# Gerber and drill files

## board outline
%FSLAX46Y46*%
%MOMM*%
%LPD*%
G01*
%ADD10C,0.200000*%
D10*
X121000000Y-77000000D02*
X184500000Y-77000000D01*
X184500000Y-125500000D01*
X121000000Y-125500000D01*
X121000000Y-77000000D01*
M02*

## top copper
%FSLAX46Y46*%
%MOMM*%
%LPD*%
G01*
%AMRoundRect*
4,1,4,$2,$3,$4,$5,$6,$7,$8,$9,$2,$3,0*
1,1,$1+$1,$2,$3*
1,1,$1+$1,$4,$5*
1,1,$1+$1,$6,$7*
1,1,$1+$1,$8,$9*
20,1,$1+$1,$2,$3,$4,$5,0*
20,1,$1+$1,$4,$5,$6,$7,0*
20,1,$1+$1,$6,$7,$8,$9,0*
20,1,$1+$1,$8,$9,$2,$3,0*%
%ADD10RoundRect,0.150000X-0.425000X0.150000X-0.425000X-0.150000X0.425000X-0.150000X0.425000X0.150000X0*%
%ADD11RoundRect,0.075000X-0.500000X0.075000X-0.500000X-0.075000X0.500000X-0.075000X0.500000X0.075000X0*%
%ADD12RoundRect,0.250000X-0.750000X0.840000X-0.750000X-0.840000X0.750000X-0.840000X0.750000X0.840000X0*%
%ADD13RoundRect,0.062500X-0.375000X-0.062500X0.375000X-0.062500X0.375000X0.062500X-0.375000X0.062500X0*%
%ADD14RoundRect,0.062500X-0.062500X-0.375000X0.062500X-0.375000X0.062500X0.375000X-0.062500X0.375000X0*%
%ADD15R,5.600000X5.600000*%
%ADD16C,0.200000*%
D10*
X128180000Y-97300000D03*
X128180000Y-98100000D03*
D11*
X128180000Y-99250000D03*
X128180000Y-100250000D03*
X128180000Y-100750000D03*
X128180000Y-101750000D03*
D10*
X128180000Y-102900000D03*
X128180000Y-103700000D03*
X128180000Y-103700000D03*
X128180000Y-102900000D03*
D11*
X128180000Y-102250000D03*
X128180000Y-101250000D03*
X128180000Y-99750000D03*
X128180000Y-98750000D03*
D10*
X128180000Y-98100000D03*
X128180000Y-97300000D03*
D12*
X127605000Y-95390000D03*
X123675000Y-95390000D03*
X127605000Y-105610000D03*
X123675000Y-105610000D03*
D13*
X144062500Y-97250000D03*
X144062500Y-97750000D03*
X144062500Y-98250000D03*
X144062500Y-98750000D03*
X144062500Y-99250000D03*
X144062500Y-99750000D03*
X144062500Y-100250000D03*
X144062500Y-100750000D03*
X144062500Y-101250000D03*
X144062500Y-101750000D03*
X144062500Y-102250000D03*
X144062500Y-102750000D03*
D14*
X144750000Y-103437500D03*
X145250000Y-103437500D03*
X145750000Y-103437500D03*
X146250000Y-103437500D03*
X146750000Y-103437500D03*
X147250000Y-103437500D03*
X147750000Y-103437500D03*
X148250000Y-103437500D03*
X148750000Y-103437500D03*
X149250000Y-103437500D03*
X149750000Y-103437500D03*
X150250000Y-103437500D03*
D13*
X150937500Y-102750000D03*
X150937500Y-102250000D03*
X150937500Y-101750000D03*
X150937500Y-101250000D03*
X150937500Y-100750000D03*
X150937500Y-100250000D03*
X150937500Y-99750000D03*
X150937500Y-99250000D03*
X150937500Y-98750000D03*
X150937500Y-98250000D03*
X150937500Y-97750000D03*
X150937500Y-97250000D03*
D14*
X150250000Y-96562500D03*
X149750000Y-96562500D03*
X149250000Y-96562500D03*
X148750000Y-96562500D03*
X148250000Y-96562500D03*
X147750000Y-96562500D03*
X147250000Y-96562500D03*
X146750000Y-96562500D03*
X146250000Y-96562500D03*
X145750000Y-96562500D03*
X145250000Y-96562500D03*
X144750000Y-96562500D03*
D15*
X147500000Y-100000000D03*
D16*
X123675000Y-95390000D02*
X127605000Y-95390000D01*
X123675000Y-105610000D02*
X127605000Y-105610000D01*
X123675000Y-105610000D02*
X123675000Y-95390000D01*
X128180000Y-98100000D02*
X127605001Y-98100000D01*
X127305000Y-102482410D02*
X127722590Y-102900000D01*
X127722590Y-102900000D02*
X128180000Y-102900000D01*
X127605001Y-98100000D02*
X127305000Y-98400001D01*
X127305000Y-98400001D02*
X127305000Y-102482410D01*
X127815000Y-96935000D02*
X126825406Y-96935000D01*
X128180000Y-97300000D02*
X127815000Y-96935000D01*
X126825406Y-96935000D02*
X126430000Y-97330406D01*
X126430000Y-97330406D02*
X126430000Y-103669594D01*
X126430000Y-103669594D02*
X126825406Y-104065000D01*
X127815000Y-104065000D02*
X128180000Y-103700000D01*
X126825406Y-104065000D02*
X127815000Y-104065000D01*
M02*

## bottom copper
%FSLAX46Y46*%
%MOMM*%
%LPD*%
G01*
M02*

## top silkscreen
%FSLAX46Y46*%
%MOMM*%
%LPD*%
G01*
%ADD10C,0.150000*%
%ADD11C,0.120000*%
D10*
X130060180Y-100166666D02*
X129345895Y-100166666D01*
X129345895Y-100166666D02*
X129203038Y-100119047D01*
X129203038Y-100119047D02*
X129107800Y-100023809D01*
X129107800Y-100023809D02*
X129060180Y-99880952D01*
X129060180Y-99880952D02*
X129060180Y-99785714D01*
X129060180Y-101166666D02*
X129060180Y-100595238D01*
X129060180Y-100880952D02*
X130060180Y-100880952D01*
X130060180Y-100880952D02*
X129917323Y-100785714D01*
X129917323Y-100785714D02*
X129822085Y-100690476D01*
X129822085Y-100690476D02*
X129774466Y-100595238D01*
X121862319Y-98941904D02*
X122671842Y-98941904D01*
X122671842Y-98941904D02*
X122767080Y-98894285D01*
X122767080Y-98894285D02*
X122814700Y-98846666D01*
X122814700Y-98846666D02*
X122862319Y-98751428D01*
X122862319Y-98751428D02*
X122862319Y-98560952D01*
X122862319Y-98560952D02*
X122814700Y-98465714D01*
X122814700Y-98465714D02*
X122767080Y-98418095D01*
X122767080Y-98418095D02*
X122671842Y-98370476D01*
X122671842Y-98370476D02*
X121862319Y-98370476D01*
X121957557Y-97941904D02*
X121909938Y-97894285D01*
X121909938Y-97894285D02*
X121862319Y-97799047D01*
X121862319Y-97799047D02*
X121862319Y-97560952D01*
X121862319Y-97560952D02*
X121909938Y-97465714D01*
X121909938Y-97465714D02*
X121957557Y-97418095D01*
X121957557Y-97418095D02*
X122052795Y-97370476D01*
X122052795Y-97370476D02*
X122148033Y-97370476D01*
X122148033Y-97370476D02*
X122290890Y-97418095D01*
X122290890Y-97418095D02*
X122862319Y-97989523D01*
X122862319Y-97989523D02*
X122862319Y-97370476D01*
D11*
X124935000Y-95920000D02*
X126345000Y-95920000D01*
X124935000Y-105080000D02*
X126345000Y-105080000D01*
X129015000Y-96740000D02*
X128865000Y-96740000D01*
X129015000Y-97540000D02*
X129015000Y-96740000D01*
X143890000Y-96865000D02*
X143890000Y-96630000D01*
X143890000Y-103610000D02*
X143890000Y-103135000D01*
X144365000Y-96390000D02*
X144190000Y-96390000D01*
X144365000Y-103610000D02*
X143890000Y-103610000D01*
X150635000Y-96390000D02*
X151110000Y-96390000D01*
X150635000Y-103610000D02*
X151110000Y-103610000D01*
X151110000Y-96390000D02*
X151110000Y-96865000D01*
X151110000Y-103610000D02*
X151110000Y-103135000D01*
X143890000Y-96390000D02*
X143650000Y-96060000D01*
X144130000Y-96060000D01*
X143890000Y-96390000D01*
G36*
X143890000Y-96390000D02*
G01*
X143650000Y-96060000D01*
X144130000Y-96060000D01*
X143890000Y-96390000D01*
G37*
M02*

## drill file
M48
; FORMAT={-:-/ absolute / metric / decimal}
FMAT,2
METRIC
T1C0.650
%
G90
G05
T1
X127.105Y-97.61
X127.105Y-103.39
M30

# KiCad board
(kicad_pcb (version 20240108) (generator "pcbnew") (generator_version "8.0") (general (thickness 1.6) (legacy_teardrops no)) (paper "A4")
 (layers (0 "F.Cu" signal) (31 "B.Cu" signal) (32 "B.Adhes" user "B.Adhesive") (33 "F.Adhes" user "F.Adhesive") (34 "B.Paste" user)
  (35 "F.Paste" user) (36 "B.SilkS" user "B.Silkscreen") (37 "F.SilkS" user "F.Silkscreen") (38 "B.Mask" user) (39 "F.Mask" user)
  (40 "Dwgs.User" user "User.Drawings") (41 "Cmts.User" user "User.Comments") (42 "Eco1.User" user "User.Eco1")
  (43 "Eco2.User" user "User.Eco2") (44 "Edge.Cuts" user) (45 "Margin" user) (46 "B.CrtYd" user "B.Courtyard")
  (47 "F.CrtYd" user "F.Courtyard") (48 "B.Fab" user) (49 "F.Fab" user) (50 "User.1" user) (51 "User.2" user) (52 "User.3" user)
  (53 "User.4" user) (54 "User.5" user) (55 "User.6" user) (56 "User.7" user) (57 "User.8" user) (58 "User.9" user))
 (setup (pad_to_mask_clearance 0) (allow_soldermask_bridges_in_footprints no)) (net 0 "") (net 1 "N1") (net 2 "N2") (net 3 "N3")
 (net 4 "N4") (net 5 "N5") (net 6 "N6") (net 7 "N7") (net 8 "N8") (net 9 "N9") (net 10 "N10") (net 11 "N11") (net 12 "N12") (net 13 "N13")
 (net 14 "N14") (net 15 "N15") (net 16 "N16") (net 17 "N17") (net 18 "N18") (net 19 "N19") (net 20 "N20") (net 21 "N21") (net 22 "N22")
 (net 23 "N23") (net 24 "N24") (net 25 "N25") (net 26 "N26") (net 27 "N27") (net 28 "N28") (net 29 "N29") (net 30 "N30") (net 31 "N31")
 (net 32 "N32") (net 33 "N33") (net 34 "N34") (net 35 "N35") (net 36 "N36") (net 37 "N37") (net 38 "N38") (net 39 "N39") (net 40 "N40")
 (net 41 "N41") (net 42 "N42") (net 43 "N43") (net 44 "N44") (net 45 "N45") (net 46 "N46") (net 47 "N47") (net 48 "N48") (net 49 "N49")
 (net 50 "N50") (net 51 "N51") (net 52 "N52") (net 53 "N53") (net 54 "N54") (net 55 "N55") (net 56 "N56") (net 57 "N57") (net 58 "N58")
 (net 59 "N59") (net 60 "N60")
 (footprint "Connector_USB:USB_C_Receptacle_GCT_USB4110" (layer "F.Cu") (at 124.5 100.5 -90)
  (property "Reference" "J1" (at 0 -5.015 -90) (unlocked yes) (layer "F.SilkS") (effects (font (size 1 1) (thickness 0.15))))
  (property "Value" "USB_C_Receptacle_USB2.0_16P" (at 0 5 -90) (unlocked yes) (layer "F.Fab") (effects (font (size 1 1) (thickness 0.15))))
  (fp_line (start -4.58 -0.435) (end -4.58 -1.845) (stroke (width 0.12) (type default)) (layer "F.SilkS"))
  (fp_line (start 4.58 -0.435) (end 4.58 -1.845) (stroke (width 0.12) (type default)) (layer "F.SilkS"))
  (fp_line (start -3.76 -4.515) (end -3.76 -4.365) (stroke (width 0.12) (type default)) (layer "F.SilkS"))
  (fp_line (start -2.96 -4.515) (end -3.76 -4.515) (stroke (width 0.12) (type default)) (layer "F.SilkS"))
  (pad "" np_thru_hole circle (at -2.89 -2.605 270) (size 0.65 0.65) (drill 0.65) (layers "F&B.Cu" "*.Mask"))
  (pad "" np_thru_hole circle (at 2.89 -2.605 270) (size 0.65 0.65) (drill 0.65) (layers "F&B.Cu" "*.Mask"))
  (pad "A1" smd roundrect (at -3.2 -3.68 270) (size 0.6 1.15) (layers "F.Cu" "F.Paste" "F.Mask") (roundrect_rratio 0.25) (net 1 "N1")
   (thermal_bridge_angle 45))
  (pad "A4" smd roundrect (at -2.4 -3.68 270) (size 0.6 1.15) (layers "F.Cu" "F.Paste" "F.Mask") (roundrect_rratio 0.25) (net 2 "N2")
   (thermal_bridge_angle 45))
  (pad "A5" smd roundrect (at -1.25 -3.68 270) (size 0.3 1.15) (layers "F.Cu" "F.Paste" "F.Mask") (roundrect_rratio 0.25) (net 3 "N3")
   (thermal_bridge_angle 45))
  (pad "A6" smd roundrect (at -0.25 -3.68 270) (size 0.3 1.15) (layers "F.Cu" "F.Paste" "F.Mask") (roundrect_rratio 0.25) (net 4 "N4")
   (thermal_bridge_angle 45))
  (pad "A7" smd roundrect (at 0.25 -3.68 270) (size 0.3 1.15) (layers "F.Cu" "F.Paste" "F.Mask") (roundrect_rratio 0.25) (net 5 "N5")
   (thermal_bridge_angle 45))
  (pad "A8" smd roundrect (at 1.25 -3.68 270) (size 0.3 1.15) (layers "F.Cu" "F.Paste" "F.Mask") (roundrect_rratio 0.25) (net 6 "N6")
   (thermal_bridge_angle 45))
  (pad "A9" smd roundrect (at 2.4 -3.68 270) (size 0.6 1.15) (layers "F.Cu" "F.Paste" "F.Mask") (roundrect_rratio 0.25) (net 2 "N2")
   (thermal_bridge_angle 45))
  (pad "A12" smd roundrect (at 3.2 -3.68 270) (size 0.6 1.15) (layers "F.Cu" "F.Paste" "F.Mask") (roundrect_rratio 0.25) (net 1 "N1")
   (thermal_bridge_angle 45))
  (pad "B1" smd roundrect (at 3.2 -3.68 270) (size 0.6 1.15) (layers "F.Cu" "F.Paste" "F.Mask") (roundrect_rratio 0.25) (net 1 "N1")
   (thermal_bridge_angle 45))
  (pad "B4" smd roundrect (at 2.4 -3.68 270) (size 0.6 1.15) (layers "F.Cu" "F.Paste" "F.Mask") (roundrect_rratio 0.25) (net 2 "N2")
   (thermal_bridge_angle 45))
  (pad "B5" smd roundrect (at 1.75 -3.68 270) (size 0.3 1.15) (layers "F.Cu" "F.Paste" "F.Mask") (roundrect_rratio 0.25) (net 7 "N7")
   (thermal_bridge_angle 45))
  (pad "B6" smd roundrect (at 0.75 -3.68 270) (size 0.3 1.15) (layers "F.Cu" "F.Paste" "F.Mask") (roundrect_rratio 0.25) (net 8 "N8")
   (thermal_bridge_angle 45))
  (pad "B7" smd roundrect (at -0.75 -3.68 270) (size 0.3 1.15) (layers "F.Cu" "F.Paste" "F.Mask") (roundrect_rratio 0.25) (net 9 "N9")
   (thermal_bridge_angle 45))
  (pad "B8" smd roundrect (at -1.75 -3.68 270) (size 0.3 1.15) (layers "F.Cu" "F.Paste" "F.Mask") (roundrect_rratio 0.25) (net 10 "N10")
   (thermal_bridge_angle 45))
  (pad "B9" smd roundrect (at -2.4 -3.68 270) (size 0.6 1.15) (layers "F.Cu" "F.Paste" "F.Mask") (roundrect_rratio 0.25) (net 2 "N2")
   (thermal_bridge_angle 45))
  (pad "B12" smd roundrect (at -3.2 -3.68 270) (size 0.6 1.15) (layers "F.Cu" "F.Paste" "F.Mask") (roundrect_rratio 0.25) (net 1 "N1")
   (thermal_bridge_angle 45))
  (pad "S1" smd roundrect (at -5.11 -3.105 270) (size 2.18 2) (layers "F.Cu" "F.Paste" "F.Mask") (roundrect_rratio 0.125) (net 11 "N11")
   (thermal_bridge_angle 45))
  (pad "S1" smd roundrect (at -5.11 0.825 270) (size 2.18 2) (layers "F.Cu" "F.Paste" "F.Mask") (roundrect_rratio 0.125) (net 11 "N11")
   (thermal_bridge_angle 45))
  (pad "S1" smd roundrect (at 5.11 -3.105 270) (size 2.18 2) (layers "F.Cu" "F.Paste" "F.Mask") (roundrect_rratio 0.125) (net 11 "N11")
   (thermal_bridge_angle 45))
  (pad "S1" smd roundrect (at 5.11 0.825 270) (size 2.18 2) (layers "F.Cu" "F.Paste" "F.Mask") (roundrect_rratio 0.125) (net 11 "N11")
   (thermal_bridge_angle 45)))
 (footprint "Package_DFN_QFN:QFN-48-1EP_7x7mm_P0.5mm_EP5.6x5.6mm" (layer "F.Cu") (at 147.5 100)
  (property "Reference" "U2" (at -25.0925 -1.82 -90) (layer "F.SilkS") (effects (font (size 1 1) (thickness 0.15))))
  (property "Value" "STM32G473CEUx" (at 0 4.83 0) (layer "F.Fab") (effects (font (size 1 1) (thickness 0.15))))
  (fp_line (start -3.61 -3.135) (end -3.61 -3.37) (stroke (width 0.12) (type solid)) (layer "F.SilkS"))
  (fp_line (start -3.61 3.61) (end -3.61 3.135) (stroke (width 0.12) (type solid)) (layer "F.SilkS"))
  (fp_line (start -3.135 -3.61) (end -3.31 -3.61) (stroke (width 0.12) (type solid)) (layer "F.SilkS"))
  (fp_line (start -3.135 3.61) (end -3.61 3.61) (stroke (width 0.12) (type solid)) (layer "F.SilkS"))
  (fp_line (start 3.135 -3.61) (end 3.61 -3.61) (stroke (width 0.12) (type solid)) (layer "F.SilkS"))
  (fp_line (start 3.135 3.61) (end 3.61 3.61) (stroke (width 0.12) (type solid)) (layer "F.SilkS"))
  (fp_line (start 3.61 -3.61) (end 3.61 -3.135) (stroke (width 0.12) (type solid)) (layer "F.SilkS"))
  (fp_line (start 3.61 3.61) (end 3.61 3.135) (stroke (width 0.12) (type solid)) (layer "F.SilkS"))
  (fp_poly
   (pts (xy -3.61 -3.61) (xy -3.85 -3.94) (xy -3.37 -3.94) (xy -3.61 -3.61)) (stroke (width 0.12) (type solid)) (fill solid)
   (layer "F.SilkS"))
  (pad "" smd roundrect (at -2.1 -2.1) (size 1.13 1.13) (layers "F.Paste") (roundrect_rratio 0.221239))
  (pad "" smd roundrect (at -2.1 -0.7) (size 1.13 1.13) (layers "F.Paste") (roundrect_rratio 0.221239))
  (pad "" smd roundrect (at -2.1 0.7) (size 1.13 1.13) (layers "F.Paste") (roundrect_rratio 0.221239))
  (pad "" smd roundrect (at -2.1 2.1) (size 1.13 1.13) (layers "F.Paste") (roundrect_rratio 0.221239))
  (pad "" smd roundrect (at -0.7 -2.1) (size 1.13 1.13) (layers "F.Paste") (roundrect_rratio 0.221239))
  (pad "" smd roundrect (at -0.7 -0.7) (size 1.13 1.13) (layers "F.Paste") (roundrect_rratio 0.221239))
  (pad "" smd roundrect (at -0.7 0.7) (size 1.13 1.13) (layers "F.Paste") (roundrect_rratio 0.221239))
  (pad "" smd roundrect (at -0.7 2.1) (size 1.13 1.13) (layers "F.Paste") (roundrect_rratio 0.221239))
  (pad "" smd roundrect (at 0.7 -2.1) (size 1.13 1.13) (layers "F.Paste") (roundrect_rratio 0.221239))
  (pad "" smd roundrect (at 0.7 -0.7) (size 1.13 1.13) (layers "F.Paste") (roundrect_rratio 0.221239))
  (pad "" smd roundrect (at 0.7 0.7) (size 1.13 1.13) (layers "F.Paste") (roundrect_rratio 0.221239))
  (pad "" smd roundrect (at 0.7 2.1) (size 1.13 1.13) (layers "F.Paste") (roundrect_rratio 0.221239))
  (pad "" smd roundrect (at 2.1 -2.1) (size 1.13 1.13) (layers "F.Paste") (roundrect_rratio 0.221239))
  (pad "" smd roundrect (at 2.1 -0.7) (size 1.13 1.13) (layers "F.Paste") (roundrect_rratio 0.221239))
  (pad "" smd roundrect (at 2.1 0.7) (size 1.13 1.13) (layers "F.Paste") (roundrect_rratio 0.221239))
  (pad "" smd roundrect (at 2.1 2.1) (size 1.13 1.13) (layers "F.Paste") (roundrect_rratio 0.221239))
  (pad "1" smd roundrect (at -3.4375 -2.75) (size 0.875 0.25) (layers "F.Cu" "F.Paste" "F.Mask") (roundrect_rratio 0.25) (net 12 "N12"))
  (pad "2" smd roundrect (at -3.4375 -2.25) (size 0.875 0.25) (layers "F.Cu" "F.Paste" "F.Mask") (roundrect_rratio 0.25) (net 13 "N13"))
  (pad "3" smd roundrect (at -3.4375 -1.75) (size 0.875 0.25) (layers "F.Cu" "F.Paste" "F.Mask") (roundrect_rratio 0.25) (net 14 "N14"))
  (pad "4" smd roundrect (at -3.4375 -1.25) (size 0.875 0.25) (layers "F.Cu" "F.Paste" "F.Mask") (roundrect_rratio 0.25) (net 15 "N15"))
  (pad "5" smd roundrect (at -3.4375 -0.75) (size 0.875 0.25) (layers "F.Cu" "F.Paste" "F.Mask") (roundrect_rratio 0.25) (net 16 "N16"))
  (pad "6" smd roundrect (at -3.4375 -0.25) (size 0.875 0.25) (layers "F.Cu" "F.Paste" "F.Mask") (roundrect_rratio 0.25) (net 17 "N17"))
  (pad "7" smd roundrect (at -3.4375 0.25) (size 0.875 0.25) (layers "F.Cu" "F.Paste" "F.Mask") (roundrect_rratio 0.25) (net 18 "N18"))
  (pad "8" smd roundrect (at -3.4375 0.75) (size 0.875 0.25) (layers "F.Cu" "F.Paste" "F.Mask") (roundrect_rratio 0.25) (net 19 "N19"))
  (pad "9" smd roundrect (at -3.4375 1.25) (size 0.875 0.25) (layers "F.Cu" "F.Paste" "F.Mask") (roundrect_rratio 0.25) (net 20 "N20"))
  (pad "10" smd roundrect (at -3.4375 1.75) (size 0.875 0.25) (layers "F.Cu" "F.Paste" "F.Mask") (roundrect_rratio 0.25) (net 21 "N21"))
  (pad "11" smd roundrect (at -3.4375 2.25) (size 0.875 0.25) (layers "F.Cu" "F.Paste" "F.Mask") (roundrect_rratio 0.25) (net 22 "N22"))
  (pad "12" smd roundrect (at -3.4375 2.75) (size 0.875 0.25) (layers "F.Cu" "F.Paste" "F.Mask") (roundrect_rratio 0.25) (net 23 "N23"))
  (pad "13" smd roundrect (at -2.75 3.4375) (size 0.25 0.875) (layers "F.Cu" "F.Paste" "F.Mask") (roundrect_rratio 0.25) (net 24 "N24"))
  (pad "14" smd roundrect (at -2.25 3.4375) (size 0.25 0.875) (layers "F.Cu" "F.Paste" "F.Mask") (roundrect_rratio 0.25) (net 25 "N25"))
  (pad "15" smd roundrect (at -1.75 3.4375) (size 0.25 0.875) (layers "F.Cu" "F.Paste" "F.Mask") (roundrect_rratio 0.25) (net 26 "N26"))
  (pad "16" smd roundrect (at -1.25 3.4375) (size 0.25 0.875) (layers "F.Cu" "F.Paste" "F.Mask") (roundrect_rratio 0.25) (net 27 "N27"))
  (pad "17" smd roundrect (at -0.75 3.4375) (size 0.25 0.875) (layers "F.Cu" "F.Paste" "F.Mask") (roundrect_rratio 0.25) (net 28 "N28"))
  (pad "18" smd roundrect (at -0.25 3.4375) (size 0.25 0.875) (layers "F.Cu" "F.Paste" "F.Mask") (roundrect_rratio 0.25) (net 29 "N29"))
  (pad "19" smd roundrect (at 0.25 3.4375) (size 0.25 0.875) (layers "F.Cu" "F.Paste" "F.Mask") (roundrect_rratio 0.25) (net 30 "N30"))
  (pad "20" smd roundrect (at 0.75 3.4375) (size 0.25 0.875) (layers "F.Cu" "F.Paste" "F.Mask") (roundrect_rratio 0.25) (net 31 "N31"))
  (pad "21" smd roundrect (at 1.25 3.4375) (size 0.25 0.875) (layers "F.Cu" "F.Paste" "F.Mask") (roundrect_rratio 0.25) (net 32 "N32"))
  (pad "22" smd roundrect (at 1.75 3.4375) (size 0.25 0.875) (layers "F.Cu" "F.Paste" "F.Mask") (roundrect_rratio 0.25) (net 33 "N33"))
  (pad "23" smd roundrect (at 2.25 3.4375) (size 0.25 0.875) (layers "F.Cu" "F.Paste" "F.Mask") (roundrect_rratio 0.25) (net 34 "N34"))
  (pad "24" smd roundrect (at 2.75 3.4375) (size 0.25 0.875) (layers "F.Cu" "F.Paste" "F.Mask") (roundrect_rratio 0.25) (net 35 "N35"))
  (pad "25" smd roundrect (at 3.4375 2.75) (size 0.875 0.25) (layers "F.Cu" "F.Paste" "F.Mask") (roundrect_rratio 0.25) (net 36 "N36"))
  (pad "26" smd roundrect (at 3.4375 2.25) (size 0.875 0.25) (layers "F.Cu" "F.Paste" "F.Mask") (roundrect_rratio 0.25) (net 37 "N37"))
  (pad "27" smd roundrect (at 3.4375 1.75) (size 0.875 0.25) (layers "F.Cu" "F.Paste" "F.Mask") (roundrect_rratio 0.25) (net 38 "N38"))
  (pad "28" smd roundrect (at 3.4375 1.25) (size 0.875 0.25) (layers "F.Cu" "F.Paste" "F.Mask") (roundrect_rratio 0.25) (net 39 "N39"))
  (pad "29" smd roundrect (at 3.4375 0.75) (size 0.875 0.25) (layers "F.Cu" "F.Paste" "F.Mask") (roundrect_rratio 0.25) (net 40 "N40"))
  (pad "30" smd roundrect (at 3.4375 0.25) (size 0.875 0.25) (layers "F.Cu" "F.Paste" "F.Mask") (roundrect_rratio 0.25) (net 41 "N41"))
  (pad "31" smd roundrect (at 3.4375 -0.25) (size 0.875 0.25) (layers "F.Cu" "F.Paste" "F.Mask") (roundrect_rratio 0.25) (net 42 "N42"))
  (pad "32" smd roundrect (at 3.4375 -0.75) (size 0.875 0.25) (layers "F.Cu" "F.Paste" "F.Mask") (roundrect_rratio 0.25) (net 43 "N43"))
  (pad "33" smd roundrect (at 3.4375 -1.25) (size 0.875 0.25) (layers "F.Cu" "F.Paste" "F.Mask") (roundrect_rratio 0.25) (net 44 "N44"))
  (pad "34" smd roundrect (at 3.4375 -1.75) (size 0.875 0.25) (layers "F.Cu" "F.Paste" "F.Mask") (roundrect_rratio 0.25) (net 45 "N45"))
  (pad "35" smd roundrect (at 3.4375 -2.25) (size 0.875 0.25) (layers "F.Cu" "F.Paste" "F.Mask") (roundrect_rratio 0.25) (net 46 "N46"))
  (pad "36" smd roundrect (at 3.4375 -2.75) (size 0.875 0.25) (layers "F.Cu" "F.Paste" "F.Mask") (roundrect_rratio 0.25) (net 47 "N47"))
  (pad "37" smd roundrect (at 2.75 -3.4375) (size 0.25 0.875) (layers "F.Cu" "F.Paste" "F.Mask") (roundrect_rratio 0.25) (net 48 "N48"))
  (pad "38" smd roundrect (at 2.25 -3.4375) (size 0.25 0.875) (layers "F.Cu" "F.Paste" "F.Mask") (roundrect_rratio 0.25) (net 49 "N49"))
  (pad "39" smd roundrect (at 1.75 -3.4375) (size 0.25 0.875) (layers "F.Cu" "F.Paste" "F.Mask") (roundrect_rratio 0.25) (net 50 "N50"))
  (pad "40" smd roundrect (at 1.25 -3.4375) (size 0.25 0.875) (layers "F.Cu" "F.Paste" "F.Mask") (roundrect_rratio 0.25) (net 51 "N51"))
  (pad "41" smd roundrect (at 0.75 -3.4375) (size 0.25 0.875) (layers "F.Cu" "F.Paste" "F.Mask") (roundrect_rratio 0.25) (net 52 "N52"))
  (pad "42" smd roundrect (at 0.25 -3.4375) (size 0.25 0.875) (layers "F.Cu" "F.Paste" "F.Mask") (roundrect_rratio 0.25) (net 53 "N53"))
  (pad "43" smd roundrect (at -0.25 -3.4375) (size 0.25 0.875) (layers "F.Cu" "F.Paste" "F.Mask") (roundrect_rratio 0.25) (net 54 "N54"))
  (pad "44" smd roundrect (at -0.75 -3.4375) (size 0.25 0.875) (layers "F.Cu" "F.Paste" "F.Mask") (roundrect_rratio 0.25) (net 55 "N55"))
  (pad "45" smd roundrect (at -1.25 -3.4375) (size 0.25 0.875) (layers "F.Cu" "F.Paste" "F.Mask") (roundrect_rratio 0.25) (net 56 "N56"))
  (pad "46" smd roundrect (at -1.75 -3.4375) (size 0.25 0.875) (layers "F.Cu" "F.Paste" "F.Mask") (roundrect_rratio 0.25) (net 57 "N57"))
  (pad "47" smd roundrect (at -2.25 -3.4375) (size 0.25 0.875) (layers "F.Cu" "F.Paste" "F.Mask") (roundrect_rratio 0.25) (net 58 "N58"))
  (pad "48" smd roundrect (at -2.75 -3.4375) (size 0.25 0.875) (layers "F.Cu" "F.Paste" "F.Mask") (roundrect_rratio 0.25) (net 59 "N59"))
  (pad "49" smd rect (at 0 0) (size 5.6 5.6) (layers "F.Cu" "F.Mask") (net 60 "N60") (zone_connect 2)))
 (gr_rect (start 121 77) (end 184.5 125.5) (stroke (width 0.2) (type default)) (fill none) (layer "Edge.Cuts"))
 (segment (start 123.675 95.39) (end 127.605 95.39) (width 0.2) (layer "F.Cu") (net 11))
 (segment (start 123.675 105.61) (end 127.605 105.61) (width 0.2) (layer "F.Cu") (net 11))
 (segment (start 123.675 105.61) (end 123.675 95.39) (width 0.2) (layer "F.Cu") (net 11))
 (segment (start 128.18 98.1) (end 127.605001 98.1) (width 0.2) (layer "F.Cu") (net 2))
 (segment (start 127.305 102.48241) (end 127.72259 102.9) (width 0.2) (layer "F.Cu") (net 2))
 (segment (start 127.72259 102.9) (end 128.18 102.9) (width 0.2) (layer "F.Cu") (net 2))
 (segment (start 127.605001 98.1) (end 127.305 98.400001) (width 0.2) (layer "F.Cu") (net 2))
 (segment (start 127.305 98.400001) (end 127.305 102.48241) (width 0.2) (layer "F.Cu") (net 2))
 (segment (start 127.815 96.935) (end 126.825406 96.935) (width 0.2) (layer "F.Cu") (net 1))
 (segment (start 128.18 97.3) (end 127.815 96.935) (width 0.2) (layer "F.Cu") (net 1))
 (segment (start 126.825406 96.935) (end 126.43 97.330406) (width 0.2) (layer "F.Cu") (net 1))
 (segment (start 126.43 97.330406) (end 126.43 103.669594) (width 0.2) (layer "F.Cu") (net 1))
 (segment (start 126.43 103.669594) (end 126.825406 104.065) (width 0.2) (layer "F.Cu") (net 1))
 (segment (start 127.815 104.065) (end 128.18 103.7) (width 0.2) (layer "F.Cu") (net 1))
 (segment (start 126.825406 104.065) (end 127.815 104.065) (width 0.2) (layer "F.Cu") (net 1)))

